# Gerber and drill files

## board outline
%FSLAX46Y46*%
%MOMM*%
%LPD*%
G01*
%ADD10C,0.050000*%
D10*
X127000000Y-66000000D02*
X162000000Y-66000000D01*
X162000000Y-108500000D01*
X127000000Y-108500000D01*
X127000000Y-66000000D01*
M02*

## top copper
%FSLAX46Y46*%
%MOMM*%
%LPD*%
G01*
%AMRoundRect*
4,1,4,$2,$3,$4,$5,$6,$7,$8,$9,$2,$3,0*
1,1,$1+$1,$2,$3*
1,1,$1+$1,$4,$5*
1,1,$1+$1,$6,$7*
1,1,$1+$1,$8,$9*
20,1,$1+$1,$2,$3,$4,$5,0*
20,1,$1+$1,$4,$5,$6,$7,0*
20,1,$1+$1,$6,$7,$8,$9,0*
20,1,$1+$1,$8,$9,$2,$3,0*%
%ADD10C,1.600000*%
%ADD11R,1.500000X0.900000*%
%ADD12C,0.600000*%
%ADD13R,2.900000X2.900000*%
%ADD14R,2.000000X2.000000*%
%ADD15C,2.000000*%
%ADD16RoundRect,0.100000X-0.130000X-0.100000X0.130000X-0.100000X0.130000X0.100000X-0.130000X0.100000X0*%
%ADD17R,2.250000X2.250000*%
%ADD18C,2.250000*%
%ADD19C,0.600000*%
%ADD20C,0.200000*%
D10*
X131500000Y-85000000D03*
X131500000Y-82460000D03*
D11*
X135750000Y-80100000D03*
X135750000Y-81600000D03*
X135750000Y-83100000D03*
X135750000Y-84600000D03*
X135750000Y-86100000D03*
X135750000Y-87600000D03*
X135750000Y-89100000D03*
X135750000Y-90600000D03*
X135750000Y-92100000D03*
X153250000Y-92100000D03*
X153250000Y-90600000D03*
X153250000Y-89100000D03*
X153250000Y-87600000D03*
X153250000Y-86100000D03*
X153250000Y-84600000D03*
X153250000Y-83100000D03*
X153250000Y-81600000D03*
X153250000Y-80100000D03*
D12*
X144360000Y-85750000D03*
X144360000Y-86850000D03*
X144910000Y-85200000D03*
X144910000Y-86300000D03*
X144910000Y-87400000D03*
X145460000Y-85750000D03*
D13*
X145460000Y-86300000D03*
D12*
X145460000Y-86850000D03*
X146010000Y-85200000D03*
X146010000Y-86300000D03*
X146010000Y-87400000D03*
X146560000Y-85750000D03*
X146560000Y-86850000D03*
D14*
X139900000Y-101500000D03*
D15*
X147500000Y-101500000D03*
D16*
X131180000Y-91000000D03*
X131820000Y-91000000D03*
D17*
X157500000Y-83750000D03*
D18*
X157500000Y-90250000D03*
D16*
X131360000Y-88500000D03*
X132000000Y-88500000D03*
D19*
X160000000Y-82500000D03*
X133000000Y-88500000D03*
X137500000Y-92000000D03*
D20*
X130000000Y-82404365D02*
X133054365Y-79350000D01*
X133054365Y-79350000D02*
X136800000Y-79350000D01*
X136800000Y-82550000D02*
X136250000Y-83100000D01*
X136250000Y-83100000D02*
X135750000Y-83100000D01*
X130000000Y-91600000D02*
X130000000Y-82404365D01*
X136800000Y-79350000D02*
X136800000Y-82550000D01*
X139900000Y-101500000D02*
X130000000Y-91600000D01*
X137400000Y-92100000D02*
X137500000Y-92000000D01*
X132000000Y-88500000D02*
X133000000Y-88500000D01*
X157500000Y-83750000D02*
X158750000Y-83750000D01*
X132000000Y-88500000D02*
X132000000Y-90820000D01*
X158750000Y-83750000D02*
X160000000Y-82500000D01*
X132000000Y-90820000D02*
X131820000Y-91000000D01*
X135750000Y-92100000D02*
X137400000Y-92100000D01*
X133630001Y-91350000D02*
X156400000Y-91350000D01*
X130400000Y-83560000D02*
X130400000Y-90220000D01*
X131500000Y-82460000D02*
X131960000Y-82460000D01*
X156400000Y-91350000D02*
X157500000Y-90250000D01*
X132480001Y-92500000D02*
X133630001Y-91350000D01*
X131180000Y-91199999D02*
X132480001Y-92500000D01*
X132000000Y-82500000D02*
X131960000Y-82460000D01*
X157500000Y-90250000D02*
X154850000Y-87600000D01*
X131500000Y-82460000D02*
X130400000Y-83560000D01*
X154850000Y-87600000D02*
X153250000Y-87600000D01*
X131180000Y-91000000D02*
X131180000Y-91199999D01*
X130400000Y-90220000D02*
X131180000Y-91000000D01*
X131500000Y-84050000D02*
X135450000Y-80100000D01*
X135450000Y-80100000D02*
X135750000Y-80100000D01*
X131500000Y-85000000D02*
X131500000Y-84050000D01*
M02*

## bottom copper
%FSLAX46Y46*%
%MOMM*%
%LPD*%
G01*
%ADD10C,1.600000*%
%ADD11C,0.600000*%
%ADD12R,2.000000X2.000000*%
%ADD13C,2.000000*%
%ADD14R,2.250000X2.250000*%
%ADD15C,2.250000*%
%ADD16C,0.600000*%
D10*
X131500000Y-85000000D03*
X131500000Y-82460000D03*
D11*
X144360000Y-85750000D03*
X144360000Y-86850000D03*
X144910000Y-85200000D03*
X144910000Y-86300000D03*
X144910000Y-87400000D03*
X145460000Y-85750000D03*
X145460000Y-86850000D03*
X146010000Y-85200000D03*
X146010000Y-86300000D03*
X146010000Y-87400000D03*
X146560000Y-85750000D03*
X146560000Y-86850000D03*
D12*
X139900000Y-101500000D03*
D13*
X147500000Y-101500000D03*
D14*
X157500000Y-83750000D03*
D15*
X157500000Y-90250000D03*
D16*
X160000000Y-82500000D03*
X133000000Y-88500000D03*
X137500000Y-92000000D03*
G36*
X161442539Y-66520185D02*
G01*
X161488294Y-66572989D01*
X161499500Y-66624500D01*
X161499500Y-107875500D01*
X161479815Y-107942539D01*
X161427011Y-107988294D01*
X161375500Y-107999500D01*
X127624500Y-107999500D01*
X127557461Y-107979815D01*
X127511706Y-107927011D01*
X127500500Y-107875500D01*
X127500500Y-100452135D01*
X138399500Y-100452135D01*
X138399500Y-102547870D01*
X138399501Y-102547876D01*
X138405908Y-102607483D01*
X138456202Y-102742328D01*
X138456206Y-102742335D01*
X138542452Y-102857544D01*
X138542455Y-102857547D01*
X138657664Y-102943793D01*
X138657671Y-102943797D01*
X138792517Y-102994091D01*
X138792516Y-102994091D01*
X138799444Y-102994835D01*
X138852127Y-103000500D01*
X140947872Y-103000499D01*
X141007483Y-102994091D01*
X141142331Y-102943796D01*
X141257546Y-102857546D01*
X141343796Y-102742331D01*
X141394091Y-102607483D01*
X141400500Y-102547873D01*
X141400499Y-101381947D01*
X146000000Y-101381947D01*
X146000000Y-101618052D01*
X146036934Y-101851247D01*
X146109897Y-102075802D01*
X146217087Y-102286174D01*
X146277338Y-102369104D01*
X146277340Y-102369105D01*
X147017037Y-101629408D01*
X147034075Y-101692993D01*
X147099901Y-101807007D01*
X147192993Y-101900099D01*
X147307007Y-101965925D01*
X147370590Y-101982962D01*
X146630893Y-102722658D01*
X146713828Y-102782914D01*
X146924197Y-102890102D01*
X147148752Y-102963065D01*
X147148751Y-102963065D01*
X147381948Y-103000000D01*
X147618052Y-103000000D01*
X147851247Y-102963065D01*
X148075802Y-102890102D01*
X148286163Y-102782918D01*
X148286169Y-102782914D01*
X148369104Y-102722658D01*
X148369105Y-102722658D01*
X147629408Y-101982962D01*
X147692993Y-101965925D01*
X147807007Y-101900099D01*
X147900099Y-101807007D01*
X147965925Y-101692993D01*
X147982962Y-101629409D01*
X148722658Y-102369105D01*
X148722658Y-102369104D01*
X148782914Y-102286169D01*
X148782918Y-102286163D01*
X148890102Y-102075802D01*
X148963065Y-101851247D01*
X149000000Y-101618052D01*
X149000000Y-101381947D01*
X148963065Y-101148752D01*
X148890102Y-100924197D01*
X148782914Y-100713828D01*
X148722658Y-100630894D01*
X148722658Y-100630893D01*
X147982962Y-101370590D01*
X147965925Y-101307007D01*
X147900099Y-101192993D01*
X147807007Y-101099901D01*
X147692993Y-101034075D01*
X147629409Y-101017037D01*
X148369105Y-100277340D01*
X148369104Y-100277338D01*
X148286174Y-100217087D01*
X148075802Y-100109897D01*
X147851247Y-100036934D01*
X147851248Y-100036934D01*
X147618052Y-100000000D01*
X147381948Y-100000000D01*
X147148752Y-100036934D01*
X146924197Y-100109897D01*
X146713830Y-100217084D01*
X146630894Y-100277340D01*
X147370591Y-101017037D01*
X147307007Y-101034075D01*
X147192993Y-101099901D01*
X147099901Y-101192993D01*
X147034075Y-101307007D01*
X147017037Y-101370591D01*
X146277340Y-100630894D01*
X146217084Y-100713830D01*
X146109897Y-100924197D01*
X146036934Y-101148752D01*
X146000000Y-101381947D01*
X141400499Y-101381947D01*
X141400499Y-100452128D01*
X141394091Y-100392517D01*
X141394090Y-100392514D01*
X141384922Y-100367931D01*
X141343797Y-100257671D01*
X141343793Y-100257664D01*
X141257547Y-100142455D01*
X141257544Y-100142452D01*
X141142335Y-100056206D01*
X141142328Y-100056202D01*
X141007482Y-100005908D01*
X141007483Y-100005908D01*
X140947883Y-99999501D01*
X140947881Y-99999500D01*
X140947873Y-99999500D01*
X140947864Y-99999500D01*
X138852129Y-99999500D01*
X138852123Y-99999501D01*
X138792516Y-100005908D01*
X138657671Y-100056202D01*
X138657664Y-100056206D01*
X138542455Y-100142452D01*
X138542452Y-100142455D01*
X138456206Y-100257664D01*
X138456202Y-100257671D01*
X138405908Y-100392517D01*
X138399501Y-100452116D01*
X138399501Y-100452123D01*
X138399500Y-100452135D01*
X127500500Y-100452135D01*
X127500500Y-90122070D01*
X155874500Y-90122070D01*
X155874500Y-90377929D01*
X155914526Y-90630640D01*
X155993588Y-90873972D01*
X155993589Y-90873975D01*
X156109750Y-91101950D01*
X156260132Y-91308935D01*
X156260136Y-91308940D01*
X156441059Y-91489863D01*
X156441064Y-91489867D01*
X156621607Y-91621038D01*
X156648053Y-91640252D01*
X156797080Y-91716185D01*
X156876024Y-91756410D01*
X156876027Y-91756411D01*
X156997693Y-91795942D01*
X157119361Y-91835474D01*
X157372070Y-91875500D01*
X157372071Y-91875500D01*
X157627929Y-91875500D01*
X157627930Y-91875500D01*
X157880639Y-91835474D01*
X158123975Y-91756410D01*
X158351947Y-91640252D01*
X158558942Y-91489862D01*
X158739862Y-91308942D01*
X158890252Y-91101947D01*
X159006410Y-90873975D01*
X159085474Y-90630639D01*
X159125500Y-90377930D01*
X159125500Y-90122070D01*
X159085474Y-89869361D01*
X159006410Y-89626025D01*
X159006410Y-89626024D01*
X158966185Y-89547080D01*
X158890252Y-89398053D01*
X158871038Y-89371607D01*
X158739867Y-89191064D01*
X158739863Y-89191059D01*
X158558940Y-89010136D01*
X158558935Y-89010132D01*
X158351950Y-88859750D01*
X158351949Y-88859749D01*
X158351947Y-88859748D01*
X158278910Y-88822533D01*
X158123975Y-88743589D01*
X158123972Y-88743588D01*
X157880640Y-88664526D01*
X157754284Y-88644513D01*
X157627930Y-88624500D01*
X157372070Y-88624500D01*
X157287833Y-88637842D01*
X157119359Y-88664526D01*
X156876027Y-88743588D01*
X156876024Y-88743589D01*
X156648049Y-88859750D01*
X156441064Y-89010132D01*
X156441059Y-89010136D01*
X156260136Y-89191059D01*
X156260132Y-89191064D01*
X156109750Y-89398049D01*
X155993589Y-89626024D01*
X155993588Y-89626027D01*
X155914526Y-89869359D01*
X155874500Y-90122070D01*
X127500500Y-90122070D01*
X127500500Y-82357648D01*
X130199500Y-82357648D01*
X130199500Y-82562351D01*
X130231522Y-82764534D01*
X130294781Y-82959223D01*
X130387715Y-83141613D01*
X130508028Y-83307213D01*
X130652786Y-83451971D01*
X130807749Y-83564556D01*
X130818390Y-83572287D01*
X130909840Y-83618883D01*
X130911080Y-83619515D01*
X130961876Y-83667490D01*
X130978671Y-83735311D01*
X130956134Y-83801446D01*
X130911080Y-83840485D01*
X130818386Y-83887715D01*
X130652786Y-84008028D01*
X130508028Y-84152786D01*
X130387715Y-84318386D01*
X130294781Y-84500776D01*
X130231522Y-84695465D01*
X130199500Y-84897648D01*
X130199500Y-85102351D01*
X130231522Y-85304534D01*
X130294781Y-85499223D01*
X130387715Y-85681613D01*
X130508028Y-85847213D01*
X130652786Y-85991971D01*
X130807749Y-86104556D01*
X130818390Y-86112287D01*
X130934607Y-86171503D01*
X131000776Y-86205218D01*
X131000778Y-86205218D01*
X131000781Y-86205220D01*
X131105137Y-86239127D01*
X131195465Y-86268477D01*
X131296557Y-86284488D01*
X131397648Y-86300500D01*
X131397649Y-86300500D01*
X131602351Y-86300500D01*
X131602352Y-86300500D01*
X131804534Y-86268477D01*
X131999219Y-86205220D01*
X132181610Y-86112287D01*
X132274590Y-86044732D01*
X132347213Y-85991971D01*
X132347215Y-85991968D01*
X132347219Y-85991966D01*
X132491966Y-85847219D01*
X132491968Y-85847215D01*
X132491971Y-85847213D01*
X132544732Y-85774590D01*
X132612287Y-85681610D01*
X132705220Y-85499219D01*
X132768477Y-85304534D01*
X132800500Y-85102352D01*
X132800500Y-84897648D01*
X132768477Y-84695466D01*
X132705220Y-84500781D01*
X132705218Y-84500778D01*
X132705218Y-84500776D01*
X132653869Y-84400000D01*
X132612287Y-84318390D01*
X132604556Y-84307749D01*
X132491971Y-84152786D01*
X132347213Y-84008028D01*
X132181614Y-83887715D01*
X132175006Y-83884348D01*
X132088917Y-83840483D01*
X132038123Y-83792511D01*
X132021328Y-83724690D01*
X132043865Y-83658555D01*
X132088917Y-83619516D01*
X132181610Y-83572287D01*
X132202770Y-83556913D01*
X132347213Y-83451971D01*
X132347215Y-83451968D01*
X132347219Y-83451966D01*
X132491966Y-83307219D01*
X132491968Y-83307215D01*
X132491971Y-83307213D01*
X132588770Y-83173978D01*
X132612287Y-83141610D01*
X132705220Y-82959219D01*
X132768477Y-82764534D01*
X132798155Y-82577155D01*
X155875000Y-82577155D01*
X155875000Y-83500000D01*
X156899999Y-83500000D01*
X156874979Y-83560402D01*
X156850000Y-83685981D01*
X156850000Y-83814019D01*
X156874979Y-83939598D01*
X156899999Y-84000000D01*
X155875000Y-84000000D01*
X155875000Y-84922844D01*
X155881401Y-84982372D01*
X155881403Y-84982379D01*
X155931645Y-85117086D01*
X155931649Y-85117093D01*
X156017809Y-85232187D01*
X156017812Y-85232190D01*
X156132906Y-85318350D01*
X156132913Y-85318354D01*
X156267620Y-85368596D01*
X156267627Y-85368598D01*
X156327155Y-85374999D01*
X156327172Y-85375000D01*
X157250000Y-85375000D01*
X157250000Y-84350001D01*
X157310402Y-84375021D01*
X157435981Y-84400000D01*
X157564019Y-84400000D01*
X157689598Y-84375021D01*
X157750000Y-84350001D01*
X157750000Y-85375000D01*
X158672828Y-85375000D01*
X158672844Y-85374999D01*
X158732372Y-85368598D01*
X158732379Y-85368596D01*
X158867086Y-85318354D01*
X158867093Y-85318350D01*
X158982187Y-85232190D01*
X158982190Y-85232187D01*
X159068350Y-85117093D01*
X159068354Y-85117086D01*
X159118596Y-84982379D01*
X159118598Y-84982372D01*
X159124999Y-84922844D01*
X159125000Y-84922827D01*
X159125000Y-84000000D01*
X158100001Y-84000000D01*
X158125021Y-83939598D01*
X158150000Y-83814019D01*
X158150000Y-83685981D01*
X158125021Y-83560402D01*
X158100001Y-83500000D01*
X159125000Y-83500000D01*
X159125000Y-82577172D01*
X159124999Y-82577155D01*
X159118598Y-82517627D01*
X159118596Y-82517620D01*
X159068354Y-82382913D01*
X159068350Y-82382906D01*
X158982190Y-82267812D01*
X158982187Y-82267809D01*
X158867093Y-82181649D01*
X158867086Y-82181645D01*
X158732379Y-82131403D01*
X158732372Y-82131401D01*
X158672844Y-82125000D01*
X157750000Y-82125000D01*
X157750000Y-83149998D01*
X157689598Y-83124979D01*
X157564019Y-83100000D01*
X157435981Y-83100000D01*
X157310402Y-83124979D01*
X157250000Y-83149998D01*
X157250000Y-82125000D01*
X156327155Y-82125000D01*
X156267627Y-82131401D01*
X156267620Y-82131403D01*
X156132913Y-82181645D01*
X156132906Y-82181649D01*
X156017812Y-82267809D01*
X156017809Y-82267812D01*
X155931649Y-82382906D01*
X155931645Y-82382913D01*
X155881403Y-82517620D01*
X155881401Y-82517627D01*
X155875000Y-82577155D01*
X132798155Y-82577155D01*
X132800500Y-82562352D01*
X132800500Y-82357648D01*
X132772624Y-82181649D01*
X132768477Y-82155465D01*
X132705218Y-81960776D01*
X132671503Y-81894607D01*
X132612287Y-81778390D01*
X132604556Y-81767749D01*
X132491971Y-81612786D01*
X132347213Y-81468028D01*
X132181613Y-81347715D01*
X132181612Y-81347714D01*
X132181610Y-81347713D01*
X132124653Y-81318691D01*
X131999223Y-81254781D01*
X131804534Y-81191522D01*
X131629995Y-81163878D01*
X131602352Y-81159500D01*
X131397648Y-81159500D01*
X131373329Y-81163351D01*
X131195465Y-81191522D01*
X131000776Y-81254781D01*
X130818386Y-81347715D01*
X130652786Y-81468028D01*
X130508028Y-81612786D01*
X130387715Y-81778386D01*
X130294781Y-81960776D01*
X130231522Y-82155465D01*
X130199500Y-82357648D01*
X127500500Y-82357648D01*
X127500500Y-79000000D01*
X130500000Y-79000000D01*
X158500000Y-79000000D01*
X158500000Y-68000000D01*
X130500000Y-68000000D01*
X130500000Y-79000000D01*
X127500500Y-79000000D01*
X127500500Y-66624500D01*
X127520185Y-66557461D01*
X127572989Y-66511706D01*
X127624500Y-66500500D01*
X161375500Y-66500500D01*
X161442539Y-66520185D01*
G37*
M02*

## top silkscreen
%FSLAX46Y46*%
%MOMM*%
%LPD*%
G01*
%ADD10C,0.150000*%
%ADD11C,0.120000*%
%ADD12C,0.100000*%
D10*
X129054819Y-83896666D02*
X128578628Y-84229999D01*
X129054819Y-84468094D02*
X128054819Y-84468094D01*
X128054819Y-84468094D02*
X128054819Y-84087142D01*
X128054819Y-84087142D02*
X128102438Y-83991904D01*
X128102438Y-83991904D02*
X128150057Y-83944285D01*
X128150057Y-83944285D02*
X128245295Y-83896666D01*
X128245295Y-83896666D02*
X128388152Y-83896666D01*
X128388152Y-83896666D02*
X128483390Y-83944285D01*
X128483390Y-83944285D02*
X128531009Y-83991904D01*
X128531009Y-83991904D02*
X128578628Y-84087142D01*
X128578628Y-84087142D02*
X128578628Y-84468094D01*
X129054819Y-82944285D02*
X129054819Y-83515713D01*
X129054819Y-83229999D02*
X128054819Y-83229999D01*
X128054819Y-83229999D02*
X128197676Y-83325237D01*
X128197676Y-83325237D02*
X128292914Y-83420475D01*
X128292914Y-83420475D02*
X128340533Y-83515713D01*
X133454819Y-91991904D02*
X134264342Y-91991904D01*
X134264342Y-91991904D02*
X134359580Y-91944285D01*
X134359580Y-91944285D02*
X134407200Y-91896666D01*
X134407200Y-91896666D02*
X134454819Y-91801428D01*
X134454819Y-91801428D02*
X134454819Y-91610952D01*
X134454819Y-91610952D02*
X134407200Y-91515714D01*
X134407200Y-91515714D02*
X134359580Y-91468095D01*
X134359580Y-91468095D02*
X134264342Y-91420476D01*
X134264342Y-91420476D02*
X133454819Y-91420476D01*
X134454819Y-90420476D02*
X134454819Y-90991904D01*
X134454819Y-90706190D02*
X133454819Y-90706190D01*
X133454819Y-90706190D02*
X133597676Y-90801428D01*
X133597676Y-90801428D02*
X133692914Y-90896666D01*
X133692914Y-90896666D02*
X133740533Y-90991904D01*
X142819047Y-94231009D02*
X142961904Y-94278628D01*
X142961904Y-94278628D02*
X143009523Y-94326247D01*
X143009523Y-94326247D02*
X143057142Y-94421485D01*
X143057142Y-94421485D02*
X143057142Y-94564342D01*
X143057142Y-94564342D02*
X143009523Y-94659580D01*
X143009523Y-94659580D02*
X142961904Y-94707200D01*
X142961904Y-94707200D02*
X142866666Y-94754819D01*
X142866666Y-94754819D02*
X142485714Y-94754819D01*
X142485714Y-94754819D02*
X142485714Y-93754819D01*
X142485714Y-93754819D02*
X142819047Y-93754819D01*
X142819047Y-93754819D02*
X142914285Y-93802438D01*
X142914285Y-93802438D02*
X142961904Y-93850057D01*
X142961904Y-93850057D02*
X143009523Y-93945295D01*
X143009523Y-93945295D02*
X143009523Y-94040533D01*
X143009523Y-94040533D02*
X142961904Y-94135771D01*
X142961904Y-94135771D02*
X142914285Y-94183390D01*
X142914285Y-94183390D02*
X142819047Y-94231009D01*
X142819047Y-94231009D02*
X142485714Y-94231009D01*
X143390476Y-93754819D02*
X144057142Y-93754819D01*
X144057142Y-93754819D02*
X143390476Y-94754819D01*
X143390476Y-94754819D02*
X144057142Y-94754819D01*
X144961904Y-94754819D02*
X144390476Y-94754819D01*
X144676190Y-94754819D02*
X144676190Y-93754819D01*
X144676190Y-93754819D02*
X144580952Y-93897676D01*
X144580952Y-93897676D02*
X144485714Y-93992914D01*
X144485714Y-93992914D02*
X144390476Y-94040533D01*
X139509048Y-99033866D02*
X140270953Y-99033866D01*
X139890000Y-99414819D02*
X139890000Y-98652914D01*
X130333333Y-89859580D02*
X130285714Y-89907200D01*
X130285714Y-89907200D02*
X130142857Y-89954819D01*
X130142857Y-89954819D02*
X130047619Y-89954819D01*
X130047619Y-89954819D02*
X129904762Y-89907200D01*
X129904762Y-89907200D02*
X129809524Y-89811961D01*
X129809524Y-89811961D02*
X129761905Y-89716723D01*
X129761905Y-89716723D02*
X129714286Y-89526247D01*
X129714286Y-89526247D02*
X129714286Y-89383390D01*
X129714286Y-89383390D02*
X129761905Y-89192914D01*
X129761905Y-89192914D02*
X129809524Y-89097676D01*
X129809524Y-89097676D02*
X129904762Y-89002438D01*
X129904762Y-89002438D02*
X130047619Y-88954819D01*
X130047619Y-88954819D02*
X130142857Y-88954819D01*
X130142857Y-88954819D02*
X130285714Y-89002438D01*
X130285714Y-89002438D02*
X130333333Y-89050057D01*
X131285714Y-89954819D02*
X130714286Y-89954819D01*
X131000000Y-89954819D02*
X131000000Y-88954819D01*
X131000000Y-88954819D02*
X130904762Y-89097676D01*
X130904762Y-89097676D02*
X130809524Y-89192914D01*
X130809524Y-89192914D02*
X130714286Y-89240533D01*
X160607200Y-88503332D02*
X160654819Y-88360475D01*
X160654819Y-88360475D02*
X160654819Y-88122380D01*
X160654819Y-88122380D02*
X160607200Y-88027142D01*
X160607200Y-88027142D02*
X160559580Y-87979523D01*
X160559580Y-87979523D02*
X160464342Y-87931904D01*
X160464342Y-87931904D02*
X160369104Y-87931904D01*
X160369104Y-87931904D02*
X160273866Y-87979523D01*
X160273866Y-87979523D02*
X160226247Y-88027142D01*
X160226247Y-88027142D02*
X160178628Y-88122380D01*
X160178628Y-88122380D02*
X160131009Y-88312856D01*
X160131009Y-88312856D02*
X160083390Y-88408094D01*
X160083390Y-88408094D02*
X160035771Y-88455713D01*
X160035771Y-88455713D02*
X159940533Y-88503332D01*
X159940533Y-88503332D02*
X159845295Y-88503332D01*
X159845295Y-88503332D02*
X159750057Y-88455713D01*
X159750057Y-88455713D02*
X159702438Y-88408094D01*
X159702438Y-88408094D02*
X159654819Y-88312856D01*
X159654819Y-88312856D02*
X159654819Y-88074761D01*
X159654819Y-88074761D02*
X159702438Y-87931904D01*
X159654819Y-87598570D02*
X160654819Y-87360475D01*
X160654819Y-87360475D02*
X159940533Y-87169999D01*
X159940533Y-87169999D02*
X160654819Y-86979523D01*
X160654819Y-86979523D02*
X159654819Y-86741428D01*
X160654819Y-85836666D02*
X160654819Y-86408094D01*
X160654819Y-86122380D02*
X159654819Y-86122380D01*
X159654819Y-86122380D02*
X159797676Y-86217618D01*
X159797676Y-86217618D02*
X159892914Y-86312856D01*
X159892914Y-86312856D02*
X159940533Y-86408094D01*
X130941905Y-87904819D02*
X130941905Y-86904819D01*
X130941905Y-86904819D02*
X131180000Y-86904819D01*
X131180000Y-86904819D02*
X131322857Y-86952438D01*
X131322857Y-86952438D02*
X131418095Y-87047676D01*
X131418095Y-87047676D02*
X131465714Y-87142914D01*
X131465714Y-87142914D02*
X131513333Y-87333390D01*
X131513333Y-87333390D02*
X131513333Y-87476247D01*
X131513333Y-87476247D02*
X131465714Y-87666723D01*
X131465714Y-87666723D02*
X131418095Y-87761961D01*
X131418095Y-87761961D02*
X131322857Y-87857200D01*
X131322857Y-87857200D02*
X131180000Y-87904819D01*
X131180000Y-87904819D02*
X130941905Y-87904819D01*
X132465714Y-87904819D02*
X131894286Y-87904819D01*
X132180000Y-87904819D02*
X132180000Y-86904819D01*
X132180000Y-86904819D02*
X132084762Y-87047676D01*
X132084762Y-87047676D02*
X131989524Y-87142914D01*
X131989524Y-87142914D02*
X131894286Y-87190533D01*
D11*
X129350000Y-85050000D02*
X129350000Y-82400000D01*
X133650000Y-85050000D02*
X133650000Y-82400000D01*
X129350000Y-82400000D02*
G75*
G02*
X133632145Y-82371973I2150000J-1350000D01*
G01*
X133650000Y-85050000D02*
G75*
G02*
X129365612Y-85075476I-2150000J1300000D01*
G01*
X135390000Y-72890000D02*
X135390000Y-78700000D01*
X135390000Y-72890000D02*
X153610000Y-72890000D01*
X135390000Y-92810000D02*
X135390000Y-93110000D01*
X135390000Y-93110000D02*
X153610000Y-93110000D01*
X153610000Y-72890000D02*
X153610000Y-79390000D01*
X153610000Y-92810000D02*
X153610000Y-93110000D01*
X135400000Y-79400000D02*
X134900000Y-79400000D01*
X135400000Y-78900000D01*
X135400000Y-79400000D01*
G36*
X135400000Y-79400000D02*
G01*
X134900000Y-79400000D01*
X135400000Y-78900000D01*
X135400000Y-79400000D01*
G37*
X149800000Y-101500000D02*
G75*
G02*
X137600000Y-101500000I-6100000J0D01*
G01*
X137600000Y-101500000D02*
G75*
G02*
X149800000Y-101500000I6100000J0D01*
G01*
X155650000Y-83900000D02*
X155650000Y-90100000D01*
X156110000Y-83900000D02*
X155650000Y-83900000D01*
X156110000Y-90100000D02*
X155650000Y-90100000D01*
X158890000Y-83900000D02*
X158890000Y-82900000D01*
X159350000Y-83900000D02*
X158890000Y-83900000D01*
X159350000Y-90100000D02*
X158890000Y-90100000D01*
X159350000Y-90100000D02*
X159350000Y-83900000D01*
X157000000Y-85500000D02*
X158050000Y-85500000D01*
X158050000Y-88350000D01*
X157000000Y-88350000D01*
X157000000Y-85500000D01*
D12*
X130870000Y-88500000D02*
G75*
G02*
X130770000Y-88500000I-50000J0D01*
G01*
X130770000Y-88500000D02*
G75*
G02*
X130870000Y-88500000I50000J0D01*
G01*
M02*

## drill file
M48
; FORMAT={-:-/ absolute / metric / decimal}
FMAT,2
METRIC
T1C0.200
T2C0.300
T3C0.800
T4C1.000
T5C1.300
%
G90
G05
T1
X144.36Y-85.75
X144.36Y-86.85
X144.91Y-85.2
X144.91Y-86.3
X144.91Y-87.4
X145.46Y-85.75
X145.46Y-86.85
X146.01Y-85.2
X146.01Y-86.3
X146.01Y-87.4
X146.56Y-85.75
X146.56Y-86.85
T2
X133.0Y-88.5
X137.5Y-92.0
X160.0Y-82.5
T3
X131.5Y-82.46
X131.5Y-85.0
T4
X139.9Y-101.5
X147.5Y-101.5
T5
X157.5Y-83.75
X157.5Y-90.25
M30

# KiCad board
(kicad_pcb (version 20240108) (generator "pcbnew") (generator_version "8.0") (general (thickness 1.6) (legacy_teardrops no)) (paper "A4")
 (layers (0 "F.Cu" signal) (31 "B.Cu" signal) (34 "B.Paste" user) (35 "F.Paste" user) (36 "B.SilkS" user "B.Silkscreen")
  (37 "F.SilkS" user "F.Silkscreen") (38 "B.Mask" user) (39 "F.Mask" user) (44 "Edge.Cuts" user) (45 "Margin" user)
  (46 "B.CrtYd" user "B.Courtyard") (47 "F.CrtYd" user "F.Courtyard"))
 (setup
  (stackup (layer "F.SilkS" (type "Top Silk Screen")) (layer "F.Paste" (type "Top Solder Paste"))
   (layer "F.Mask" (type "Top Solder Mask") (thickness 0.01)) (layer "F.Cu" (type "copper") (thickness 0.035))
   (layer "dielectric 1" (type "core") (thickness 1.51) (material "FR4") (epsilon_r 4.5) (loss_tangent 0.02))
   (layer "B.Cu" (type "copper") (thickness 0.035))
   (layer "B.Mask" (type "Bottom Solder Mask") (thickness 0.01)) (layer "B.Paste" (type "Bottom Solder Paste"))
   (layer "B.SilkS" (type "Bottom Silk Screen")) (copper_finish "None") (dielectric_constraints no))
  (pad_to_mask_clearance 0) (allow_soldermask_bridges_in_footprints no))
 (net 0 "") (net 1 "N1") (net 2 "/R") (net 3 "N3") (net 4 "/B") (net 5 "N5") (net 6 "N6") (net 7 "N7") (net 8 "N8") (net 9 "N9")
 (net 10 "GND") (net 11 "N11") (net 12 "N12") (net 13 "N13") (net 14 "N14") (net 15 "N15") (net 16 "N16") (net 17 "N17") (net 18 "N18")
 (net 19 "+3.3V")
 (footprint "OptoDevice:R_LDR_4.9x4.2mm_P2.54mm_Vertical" (layer "F.Cu") (at 131.5 85 90)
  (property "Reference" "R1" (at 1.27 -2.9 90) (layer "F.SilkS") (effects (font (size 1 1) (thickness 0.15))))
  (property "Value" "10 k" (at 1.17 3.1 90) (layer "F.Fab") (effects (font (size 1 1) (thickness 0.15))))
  (fp_line (start -0.05 -2.15) (end 2.6 -2.15) (stroke (width 0.12) (type solid)) (layer "F.SilkS"))
  (fp_line (start -0.05 2.15) (end 2.6 2.15) (stroke (width 0.12) (type solid)) (layer "F.SilkS"))
  (fp_arc (start 2.6 -2.15) (mid 3.788646 -0.016616) (end 2.628027 2.132145) (stroke (width 0.12) (type solid)) (layer "F.SilkS"))
  (fp_arc (start -0.05 2.15) (mid -1.262424 0.01494) (end -0.075476 -2.134388) (stroke (width 0.12) (type solid)) (layer "F.SilkS"))
  (pad "1" thru_hole circle (at 0 0 90) (size 1.6 1.6) (drill 0.8) (layers "*.Cu" "*.Mask") (remove_unused_layers no) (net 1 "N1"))
  (pad "2" thru_hole circle (at 2.54 0 90) (size 1.6 1.6) (drill 0.8) (layers "*.Cu" "*.Mask") (remove_unused_layers no) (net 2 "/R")))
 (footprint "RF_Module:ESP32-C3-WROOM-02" (layer "F.Cu") (at 144.5 86.1)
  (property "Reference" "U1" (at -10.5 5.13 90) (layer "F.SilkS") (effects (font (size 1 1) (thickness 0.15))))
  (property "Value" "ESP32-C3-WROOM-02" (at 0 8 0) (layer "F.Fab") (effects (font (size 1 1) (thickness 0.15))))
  (fp_line (start -9.11 -13.21) (end -9.11 -7.4) (stroke (width 0.12) (type solid)) (layer "F.SilkS"))
  (fp_line (start -9.11 -13.21) (end 9.11 -13.21) (stroke (width 0.12) (type solid)) (layer "F.SilkS"))
  (fp_line (start -9.11 6.71) (end -9.11 7.01) (stroke (width 0.12) (type solid)) (layer "F.SilkS"))
  (fp_line (start -9.11 7.01) (end 9.11 7.01) (stroke (width 0.12) (type solid)) (layer "F.SilkS"))
  (fp_line (start 9.11 -13.21) (end 9.11 -6.71) (stroke (width 0.12) (type solid)) (layer "F.SilkS"))
  (fp_line (start 9.11 6.71) (end 9.11 7.01) (stroke (width 0.12) (type solid)) (layer "F.SilkS"))
  (fp_poly
   (pts (xy -9.1 -6.7) (xy -9.6 -6.7) (xy -9.1 -7.2) (xy -9.1 -6.7)) (stroke (width 0.12) (type solid)) (fill solid) (layer "F.SilkS"))
  (pad "" smd rect (at -0.14 -0.9) (size 0.7 0.7) (layers "F.Paste"))
  (pad "" smd rect (at -0.14 0.2) (size 0.7 0.7) (layers "F.Paste"))
  (pad "" smd rect (at -0.14 1.3) (size 0.7 0.7) (layers "F.Paste"))
  (pad "" smd rect (at 0.96 -0.9) (size 0.7 0.7) (layers "F.Paste"))
  (pad "" smd rect (at 0.96 0.2) (size 0.7 0.7) (layers "F.Paste"))
  (pad "" smd rect (at 0.96 1.3) (size 0.7 0.7) (layers "F.Paste"))
  (pad "" smd rect (at 2.06 -0.9) (size 0.7 0.7) (layers "F.Paste"))
  (pad "" smd rect (at 2.06 0.2) (size 0.7 0.7) (layers "F.Paste"))
  (pad "" smd rect (at 2.06 1.3) (size 0.7 0.7) (layers "F.Paste"))
  (pad "1" smd rect (at -8.75 -6) (size 1.5 0.9) (layers "F.Cu" "F.Paste" "F.Mask") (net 1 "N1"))
  (pad "2" smd rect (at -8.75 -4.5) (size 1.5 0.9) (layers "F.Cu" "F.Paste" "F.Mask") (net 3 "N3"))
  (pad "3" smd rect (at -8.75 -3) (size 1.5 0.9) (layers "F.Cu" "F.Paste" "F.Mask") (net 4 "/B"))
  (pad "4" smd rect (at -8.75 -1.5) (size 1.5 0.9) (layers "F.Cu" "F.Paste" "F.Mask") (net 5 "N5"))
  (pad "5" smd rect (at -8.75 0) (size 1.5 0.9) (layers "F.Cu" "F.Paste" "F.Mask") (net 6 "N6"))
  (pad "6" smd rect (at -8.75 1.5) (size 1.5 0.9) (layers "F.Cu" "F.Paste" "F.Mask") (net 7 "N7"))
  (pad "7" smd rect (at -8.75 3) (size 1.5 0.9) (layers "F.Cu" "F.Paste" "F.Mask") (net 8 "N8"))
  (pad "8" smd rect (at -8.75 4.5) (size 1.5 0.9) (layers "F.Cu" "F.Paste" "F.Mask") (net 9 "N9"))
  (pad "9" smd rect (at -8.75 6) (size 1.5 0.9) (layers "F.Cu" "F.Paste" "F.Mask") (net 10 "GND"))
  (pad "10" smd rect (at 8.75 6) (size 1.5 0.9) (layers "F.Cu" "F.Paste" "F.Mask") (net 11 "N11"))
  (pad "11" smd rect (at 8.75 4.5) (size 1.5 0.9) (layers "F.Cu" "F.Paste" "F.Mask") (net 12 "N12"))
  (pad "12" smd rect (at 8.75 3) (size 1.5 0.9) (layers "F.Cu" "F.Paste" "F.Mask") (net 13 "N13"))
  (pad "13" smd rect (at 8.75 1.5) (size 1.5 0.9) (layers "F.Cu" "F.Paste" "F.Mask") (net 2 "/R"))
  (pad "14" smd rect (at 8.75 0) (size 1.5 0.9) (layers "F.Cu" "F.Paste" "F.Mask") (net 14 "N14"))
  (pad "15" smd rect (at 8.75 -1.5) (size 1.5 0.9) (layers "F.Cu" "F.Paste" "F.Mask") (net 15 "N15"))
  (pad "16" smd rect (at 8.75 -3) (size 1.5 0.9) (layers "F.Cu" "F.Paste" "F.Mask") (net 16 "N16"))
  (pad "17" smd rect (at 8.75 -4.5) (size 1.5 0.9) (layers "F.Cu" "F.Paste" "F.Mask") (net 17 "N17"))
  (pad "18" smd rect (at 8.75 -6) (size 1.5 0.9) (layers "F.Cu" "F.Paste" "F.Mask") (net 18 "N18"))
  (pad "19" thru_hole circle (at -0.14 -0.35) (size 0.6 0.6) (drill 0.2) (layers "*.Cu" "F.Mask") (remove_unused_layers no) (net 10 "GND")
   (zone_connect 2))
  (pad "19" thru_hole circle (at -0.14 0.75) (size 0.6 0.6) (drill 0.2) (layers "*.Cu" "F.Mask") (remove_unused_layers no) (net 10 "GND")
   (zone_connect 2))
  (pad "19" thru_hole circle (at 0.41 -0.9) (size 0.6 0.6) (drill 0.2) (layers "*.Cu" "F.Mask") (remove_unused_layers no) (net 10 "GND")
   (zone_connect 2))
  (pad "19" thru_hole circle (at 0.41 0.2) (size 0.6 0.6) (drill 0.2) (layers "*.Cu" "F.Mask") (remove_unused_layers no) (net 10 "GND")
   (zone_connect 2))
  (pad "19" thru_hole circle (at 0.41 1.3) (size 0.6 0.6) (drill 0.2) (layers "*.Cu" "F.Mask") (remove_unused_layers no) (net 10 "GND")
   (zone_connect 2))
  (pad "19" thru_hole circle (at 0.96 -0.35) (size 0.6 0.6) (drill 0.2) (layers "*.Cu" "F.Mask") (remove_unused_layers no) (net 10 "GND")
   (zone_connect 2))
  (pad "19" smd rect (at 0.96 0.2) (size 2.9 2.9) (layers "F.Cu" "F.Mask") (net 10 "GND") (zone_connect 2))
  (pad "19" thru_hole circle (at 0.96 0.75) (size 0.6 0.6) (drill 0.2) (layers "*.Cu" "F.Mask") (remove_unused_layers no) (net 10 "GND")
   (zone_connect 2))
  (pad "19" thru_hole circle (at 1.51 -0.9) (size 0.6 0.6) (drill 0.2) (layers "*.Cu" "F.Mask") (remove_unused_layers no) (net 10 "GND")
   (zone_connect 2))
  (pad "19" thru_hole circle (at 1.51 0.2) (size 0.6 0.6) (drill 0.2) (layers "*.Cu" "F.Mask") (remove_unused_layers no) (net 10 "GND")
   (zone_connect 2))
  (pad "19" thru_hole circle (at 1.51 1.3) (size 0.6 0.6) (drill 0.2) (layers "*.Cu" "F.Mask") (remove_unused_layers no) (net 10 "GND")
   (zone_connect 2))
  (pad "19" thru_hole circle (at 2.06 -0.35) (size 0.6 0.6) (drill 0.2) (layers "*.Cu" "F.Mask") (remove_unused_layers no) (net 10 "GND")
   (zone_connect 2))
  (pad "19" thru_hole circle (at 2.06 0.75) (size 0.6 0.6) (drill 0.2) (layers "*.Cu" "F.Mask") (remove_unused_layers no) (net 10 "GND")
   (zone_connect 2))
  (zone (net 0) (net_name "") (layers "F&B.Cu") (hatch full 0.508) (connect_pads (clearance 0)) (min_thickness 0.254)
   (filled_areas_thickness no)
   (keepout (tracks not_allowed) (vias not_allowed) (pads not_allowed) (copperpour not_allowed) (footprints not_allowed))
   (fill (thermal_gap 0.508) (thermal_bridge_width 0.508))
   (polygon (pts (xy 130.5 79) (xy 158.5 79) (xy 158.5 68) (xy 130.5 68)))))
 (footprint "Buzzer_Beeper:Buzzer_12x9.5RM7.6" (layer "F.Cu") (at 139.9 101.5)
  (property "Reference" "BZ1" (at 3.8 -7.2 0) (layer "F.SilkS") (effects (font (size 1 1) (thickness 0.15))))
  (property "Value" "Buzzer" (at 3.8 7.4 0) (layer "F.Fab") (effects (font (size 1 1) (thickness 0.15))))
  (fp_circle (center 3.8 0) (end 9.9 0) (stroke (width 0.12) (type solid)) (fill none) (layer "F.SilkS"))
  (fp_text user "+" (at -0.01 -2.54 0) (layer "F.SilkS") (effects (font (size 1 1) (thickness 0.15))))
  (pad "1" thru_hole rect (at 0 0) (size 2 2) (drill 1) (layers "*.Cu" "*.Mask") (remove_unused_layers no) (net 4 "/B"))
  (pad "2" thru_hole circle (at 7.6 0) (size 2 2) (drill 1) (layers "*.Cu" "*.Mask") (remove_unused_layers no) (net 10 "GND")))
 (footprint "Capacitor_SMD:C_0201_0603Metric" (layer "F.Cu") (at 131.5 91)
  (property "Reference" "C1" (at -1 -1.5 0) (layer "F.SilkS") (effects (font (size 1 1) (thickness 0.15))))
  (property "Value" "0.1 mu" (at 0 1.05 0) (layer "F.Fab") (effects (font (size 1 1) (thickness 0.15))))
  (pad "" smd roundrect (at -0.345 0) (size 0.318 0.36) (layers "F.Paste") (roundrect_rratio 0.25))
  (pad "" smd roundrect (at 0.345 0) (size 0.318 0.36) (layers "F.Paste") (roundrect_rratio 0.25))
  (pad "1" smd roundrect (at -0.32 0) (size 0.46 0.4) (layers "F.Cu" "F.Mask") (roundrect_rratio 0.25) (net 2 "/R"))
  (pad "2" smd roundrect (at 0.32 0) (size 0.46 0.4) (layers "F.Cu" "F.Mask") (roundrect_rratio 0.25) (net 10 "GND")))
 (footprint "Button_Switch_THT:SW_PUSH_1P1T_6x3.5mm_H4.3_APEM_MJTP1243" (layer "F.Cu") (at 157.5 83.75 -90)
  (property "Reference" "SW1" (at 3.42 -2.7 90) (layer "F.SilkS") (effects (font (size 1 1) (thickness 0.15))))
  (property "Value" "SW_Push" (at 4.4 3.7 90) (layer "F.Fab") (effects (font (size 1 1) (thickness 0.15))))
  (fp_line (start 0.15 1.85) (end 6.35 1.85) (stroke (width 0.12) (type solid)) (layer "F.SilkS"))
  (fp_line (start 0.15 1.39) (end 0.15 1.85) (stroke (width 0.12) (type solid)) (layer "F.SilkS"))
  (fp_line (start 6.35 1.39) (end 6.35 1.85) (stroke (width 0.12) (type solid)) (layer "F.SilkS"))
  (fp_line (start 0.15 -1.39) (end -0.85 -1.39) (stroke (width 0.12) (type default)) (layer "F.SilkS"))
  (fp_line (start 0.15 -1.85) (end 0.15 -1.39) (stroke (width 0.12) (type default)) (layer "F.SilkS"))
  (fp_line (start 6.35 -1.85) (end 6.35 -1.39) (stroke (width 0.12) (type solid)) (layer "F.SilkS"))
  (fp_line (start 6.35 -1.85) (end 0.15 -1.85) (stroke (width 0.12) (type solid)) (layer "F.SilkS"))
  (fp_rect (start 1.75 -0.55) (end 4.6 0.5) (stroke (width 0.12) (type default)) (fill none) (layer "F.SilkS"))
  (pad "1" thru_hole rect (at 0 0) (size 2.25 2.25) (drill 1.3) (layers "*.Cu" "*.Mask") (remove_unused_layers no) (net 10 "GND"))
  (pad "2" thru_hole circle (at 6.5 0) (size 2.25 2.25) (drill 1.3) (layers "*.Cu" "*.Mask") (remove_unused_layers no) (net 2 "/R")))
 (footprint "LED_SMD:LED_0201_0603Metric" (layer "F.Cu") (at 131.68 88.5)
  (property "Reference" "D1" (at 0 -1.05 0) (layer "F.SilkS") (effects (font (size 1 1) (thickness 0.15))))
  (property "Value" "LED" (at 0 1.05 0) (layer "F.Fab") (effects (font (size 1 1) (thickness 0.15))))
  (fp_circle (center -0.86 0) (end -0.81 0) (stroke (width 0.1) (type solid)) (fill none) (layer "F.SilkS"))
  (pad "" smd roundrect (at -0.345 0) (size 0.318 0.36) (layers "F.Paste") (roundrect_rratio 0.25))
  (pad "" smd roundrect (at 0.345 0) (size 0.318 0.36) (layers "F.Paste") (roundrect_rratio 0.25))
  (pad "1" smd roundrect (at -0.32 0) (size 0.46 0.4) (layers "F.Cu" "F.Mask") (roundrect_rratio 0.25) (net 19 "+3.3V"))
  (pad "2" smd roundrect (at 0.32 0) (size 0.46 0.4) (layers "F.Cu" "F.Mask") (roundrect_rratio 0.25) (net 10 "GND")))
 (gr_rect (start 127 66) (end 162 108.5) (stroke (width 0.05) (type default)) (fill none) (layer "Edge.Cuts"))
 (segment (start 130 82.404365) (end 133.054365 79.35) (width 0.2) (layer "F.Cu") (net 4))
 (segment (start 133.054365 79.35) (end 136.8 79.35) (width 0.2) (layer "F.Cu") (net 4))
 (segment (start 136.8 82.55) (end 136.25 83.1) (width 0.2) (layer "F.Cu") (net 4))
 (segment (start 136.25 83.1) (end 135.75 83.1) (width 0.2) (layer "F.Cu") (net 4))
 (segment (start 130 91.6) (end 130 82.404365) (width 0.2) (layer "F.Cu") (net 4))
 (segment (start 136.8 79.35) (end 136.8 82.55) (width 0.2) (layer "F.Cu") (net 4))
 (segment (start 139.9 101.5) (end 130 91.6) (width 0.2) (layer "F.Cu") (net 4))
 (segment (start 137.4 92.1) (end 137.5 92) (width 0.2) (layer "F.Cu") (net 10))
 (segment (start 132 88.5) (end 133 88.5) (width 0.2) (layer "F.Cu") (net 10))
 (segment (start 157.5 83.75) (end 158.75 83.75) (width 0.2) (layer "F.Cu") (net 10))
 (segment (start 132 88.5) (end 132 90.82) (width 0.2) (layer "F.Cu") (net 10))
 (segment (start 158.75 83.75) (end 160 82.5) (width 0.2) (layer "F.Cu") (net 10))
 (segment (start 132 90.82) (end 131.82 91) (width 0.2) (layer "F.Cu") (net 10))
 (segment (start 135.75 92.1) (end 137.4 92.1) (width 0.2) (layer "F.Cu") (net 10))
 (via (at 160 82.5) (size 0.6) (drill 0.3) (layers "F.Cu" "B.Cu") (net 10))
 (via (at 133 88.5) (size 0.6) (drill 0.3) (layers "F.Cu" "B.Cu") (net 10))
 (via (at 137.5 92) (size 0.6) (drill 0.3) (layers "F.Cu" "B.Cu") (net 10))
 (segment (start 133.630001 91.35) (end 156.4 91.35) (width 0.2) (layer "F.Cu") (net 2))
 (segment (start 130.4 83.56) (end 130.4 90.22) (width 0.2) (layer "F.Cu") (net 2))
 (segment (start 131.5 82.46) (end 131.96 82.46) (width 0.2) (layer "F.Cu") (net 2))
 (segment (start 156.4 91.35) (end 157.5 90.25) (width 0.2) (layer "F.Cu") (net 2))
 (segment (start 132.480001 92.5) (end 133.630001 91.35) (width 0.2) (layer "F.Cu") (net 2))
 (segment (start 131.18 91.199999) (end 132.480001 92.5) (width 0.2) (layer "F.Cu") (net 2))
 (segment (start 132 82.5) (end 131.96 82.46) (width 0.2) (layer "F.Cu") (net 2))
 (segment (start 157.5 90.25) (end 154.85 87.6) (width 0.2) (layer "F.Cu") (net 2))
 (segment (start 131.5 82.46) (end 130.4 83.56) (width 0.2) (layer "F.Cu") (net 2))
 (segment (start 154.85 87.6) (end 153.25 87.6) (width 0.2) (layer "F.Cu") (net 2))
 (segment (start 131.18 91) (end 131.18 91.199999) (width 0.2) (layer "F.Cu") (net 2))
 (segment (start 130.4 90.22) (end 131.18 91) (width 0.2) (layer "F.Cu") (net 2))
 (segment (start 131.5 84.05) (end 135.45 80.1) (width 0.2) (layer "F.Cu") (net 1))
 (segment (start 135.45 80.1) (end 135.75 80.1) (width 0.2) (layer "F.Cu") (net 1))
 (segment (start 131.5 85) (end 131.5 84.05) (width 0.2) (layer "F.Cu") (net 1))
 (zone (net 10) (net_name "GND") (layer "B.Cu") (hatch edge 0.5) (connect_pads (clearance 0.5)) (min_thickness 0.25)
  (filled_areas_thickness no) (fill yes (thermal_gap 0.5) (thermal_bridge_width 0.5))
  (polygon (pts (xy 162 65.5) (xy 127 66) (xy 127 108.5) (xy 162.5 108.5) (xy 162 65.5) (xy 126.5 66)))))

